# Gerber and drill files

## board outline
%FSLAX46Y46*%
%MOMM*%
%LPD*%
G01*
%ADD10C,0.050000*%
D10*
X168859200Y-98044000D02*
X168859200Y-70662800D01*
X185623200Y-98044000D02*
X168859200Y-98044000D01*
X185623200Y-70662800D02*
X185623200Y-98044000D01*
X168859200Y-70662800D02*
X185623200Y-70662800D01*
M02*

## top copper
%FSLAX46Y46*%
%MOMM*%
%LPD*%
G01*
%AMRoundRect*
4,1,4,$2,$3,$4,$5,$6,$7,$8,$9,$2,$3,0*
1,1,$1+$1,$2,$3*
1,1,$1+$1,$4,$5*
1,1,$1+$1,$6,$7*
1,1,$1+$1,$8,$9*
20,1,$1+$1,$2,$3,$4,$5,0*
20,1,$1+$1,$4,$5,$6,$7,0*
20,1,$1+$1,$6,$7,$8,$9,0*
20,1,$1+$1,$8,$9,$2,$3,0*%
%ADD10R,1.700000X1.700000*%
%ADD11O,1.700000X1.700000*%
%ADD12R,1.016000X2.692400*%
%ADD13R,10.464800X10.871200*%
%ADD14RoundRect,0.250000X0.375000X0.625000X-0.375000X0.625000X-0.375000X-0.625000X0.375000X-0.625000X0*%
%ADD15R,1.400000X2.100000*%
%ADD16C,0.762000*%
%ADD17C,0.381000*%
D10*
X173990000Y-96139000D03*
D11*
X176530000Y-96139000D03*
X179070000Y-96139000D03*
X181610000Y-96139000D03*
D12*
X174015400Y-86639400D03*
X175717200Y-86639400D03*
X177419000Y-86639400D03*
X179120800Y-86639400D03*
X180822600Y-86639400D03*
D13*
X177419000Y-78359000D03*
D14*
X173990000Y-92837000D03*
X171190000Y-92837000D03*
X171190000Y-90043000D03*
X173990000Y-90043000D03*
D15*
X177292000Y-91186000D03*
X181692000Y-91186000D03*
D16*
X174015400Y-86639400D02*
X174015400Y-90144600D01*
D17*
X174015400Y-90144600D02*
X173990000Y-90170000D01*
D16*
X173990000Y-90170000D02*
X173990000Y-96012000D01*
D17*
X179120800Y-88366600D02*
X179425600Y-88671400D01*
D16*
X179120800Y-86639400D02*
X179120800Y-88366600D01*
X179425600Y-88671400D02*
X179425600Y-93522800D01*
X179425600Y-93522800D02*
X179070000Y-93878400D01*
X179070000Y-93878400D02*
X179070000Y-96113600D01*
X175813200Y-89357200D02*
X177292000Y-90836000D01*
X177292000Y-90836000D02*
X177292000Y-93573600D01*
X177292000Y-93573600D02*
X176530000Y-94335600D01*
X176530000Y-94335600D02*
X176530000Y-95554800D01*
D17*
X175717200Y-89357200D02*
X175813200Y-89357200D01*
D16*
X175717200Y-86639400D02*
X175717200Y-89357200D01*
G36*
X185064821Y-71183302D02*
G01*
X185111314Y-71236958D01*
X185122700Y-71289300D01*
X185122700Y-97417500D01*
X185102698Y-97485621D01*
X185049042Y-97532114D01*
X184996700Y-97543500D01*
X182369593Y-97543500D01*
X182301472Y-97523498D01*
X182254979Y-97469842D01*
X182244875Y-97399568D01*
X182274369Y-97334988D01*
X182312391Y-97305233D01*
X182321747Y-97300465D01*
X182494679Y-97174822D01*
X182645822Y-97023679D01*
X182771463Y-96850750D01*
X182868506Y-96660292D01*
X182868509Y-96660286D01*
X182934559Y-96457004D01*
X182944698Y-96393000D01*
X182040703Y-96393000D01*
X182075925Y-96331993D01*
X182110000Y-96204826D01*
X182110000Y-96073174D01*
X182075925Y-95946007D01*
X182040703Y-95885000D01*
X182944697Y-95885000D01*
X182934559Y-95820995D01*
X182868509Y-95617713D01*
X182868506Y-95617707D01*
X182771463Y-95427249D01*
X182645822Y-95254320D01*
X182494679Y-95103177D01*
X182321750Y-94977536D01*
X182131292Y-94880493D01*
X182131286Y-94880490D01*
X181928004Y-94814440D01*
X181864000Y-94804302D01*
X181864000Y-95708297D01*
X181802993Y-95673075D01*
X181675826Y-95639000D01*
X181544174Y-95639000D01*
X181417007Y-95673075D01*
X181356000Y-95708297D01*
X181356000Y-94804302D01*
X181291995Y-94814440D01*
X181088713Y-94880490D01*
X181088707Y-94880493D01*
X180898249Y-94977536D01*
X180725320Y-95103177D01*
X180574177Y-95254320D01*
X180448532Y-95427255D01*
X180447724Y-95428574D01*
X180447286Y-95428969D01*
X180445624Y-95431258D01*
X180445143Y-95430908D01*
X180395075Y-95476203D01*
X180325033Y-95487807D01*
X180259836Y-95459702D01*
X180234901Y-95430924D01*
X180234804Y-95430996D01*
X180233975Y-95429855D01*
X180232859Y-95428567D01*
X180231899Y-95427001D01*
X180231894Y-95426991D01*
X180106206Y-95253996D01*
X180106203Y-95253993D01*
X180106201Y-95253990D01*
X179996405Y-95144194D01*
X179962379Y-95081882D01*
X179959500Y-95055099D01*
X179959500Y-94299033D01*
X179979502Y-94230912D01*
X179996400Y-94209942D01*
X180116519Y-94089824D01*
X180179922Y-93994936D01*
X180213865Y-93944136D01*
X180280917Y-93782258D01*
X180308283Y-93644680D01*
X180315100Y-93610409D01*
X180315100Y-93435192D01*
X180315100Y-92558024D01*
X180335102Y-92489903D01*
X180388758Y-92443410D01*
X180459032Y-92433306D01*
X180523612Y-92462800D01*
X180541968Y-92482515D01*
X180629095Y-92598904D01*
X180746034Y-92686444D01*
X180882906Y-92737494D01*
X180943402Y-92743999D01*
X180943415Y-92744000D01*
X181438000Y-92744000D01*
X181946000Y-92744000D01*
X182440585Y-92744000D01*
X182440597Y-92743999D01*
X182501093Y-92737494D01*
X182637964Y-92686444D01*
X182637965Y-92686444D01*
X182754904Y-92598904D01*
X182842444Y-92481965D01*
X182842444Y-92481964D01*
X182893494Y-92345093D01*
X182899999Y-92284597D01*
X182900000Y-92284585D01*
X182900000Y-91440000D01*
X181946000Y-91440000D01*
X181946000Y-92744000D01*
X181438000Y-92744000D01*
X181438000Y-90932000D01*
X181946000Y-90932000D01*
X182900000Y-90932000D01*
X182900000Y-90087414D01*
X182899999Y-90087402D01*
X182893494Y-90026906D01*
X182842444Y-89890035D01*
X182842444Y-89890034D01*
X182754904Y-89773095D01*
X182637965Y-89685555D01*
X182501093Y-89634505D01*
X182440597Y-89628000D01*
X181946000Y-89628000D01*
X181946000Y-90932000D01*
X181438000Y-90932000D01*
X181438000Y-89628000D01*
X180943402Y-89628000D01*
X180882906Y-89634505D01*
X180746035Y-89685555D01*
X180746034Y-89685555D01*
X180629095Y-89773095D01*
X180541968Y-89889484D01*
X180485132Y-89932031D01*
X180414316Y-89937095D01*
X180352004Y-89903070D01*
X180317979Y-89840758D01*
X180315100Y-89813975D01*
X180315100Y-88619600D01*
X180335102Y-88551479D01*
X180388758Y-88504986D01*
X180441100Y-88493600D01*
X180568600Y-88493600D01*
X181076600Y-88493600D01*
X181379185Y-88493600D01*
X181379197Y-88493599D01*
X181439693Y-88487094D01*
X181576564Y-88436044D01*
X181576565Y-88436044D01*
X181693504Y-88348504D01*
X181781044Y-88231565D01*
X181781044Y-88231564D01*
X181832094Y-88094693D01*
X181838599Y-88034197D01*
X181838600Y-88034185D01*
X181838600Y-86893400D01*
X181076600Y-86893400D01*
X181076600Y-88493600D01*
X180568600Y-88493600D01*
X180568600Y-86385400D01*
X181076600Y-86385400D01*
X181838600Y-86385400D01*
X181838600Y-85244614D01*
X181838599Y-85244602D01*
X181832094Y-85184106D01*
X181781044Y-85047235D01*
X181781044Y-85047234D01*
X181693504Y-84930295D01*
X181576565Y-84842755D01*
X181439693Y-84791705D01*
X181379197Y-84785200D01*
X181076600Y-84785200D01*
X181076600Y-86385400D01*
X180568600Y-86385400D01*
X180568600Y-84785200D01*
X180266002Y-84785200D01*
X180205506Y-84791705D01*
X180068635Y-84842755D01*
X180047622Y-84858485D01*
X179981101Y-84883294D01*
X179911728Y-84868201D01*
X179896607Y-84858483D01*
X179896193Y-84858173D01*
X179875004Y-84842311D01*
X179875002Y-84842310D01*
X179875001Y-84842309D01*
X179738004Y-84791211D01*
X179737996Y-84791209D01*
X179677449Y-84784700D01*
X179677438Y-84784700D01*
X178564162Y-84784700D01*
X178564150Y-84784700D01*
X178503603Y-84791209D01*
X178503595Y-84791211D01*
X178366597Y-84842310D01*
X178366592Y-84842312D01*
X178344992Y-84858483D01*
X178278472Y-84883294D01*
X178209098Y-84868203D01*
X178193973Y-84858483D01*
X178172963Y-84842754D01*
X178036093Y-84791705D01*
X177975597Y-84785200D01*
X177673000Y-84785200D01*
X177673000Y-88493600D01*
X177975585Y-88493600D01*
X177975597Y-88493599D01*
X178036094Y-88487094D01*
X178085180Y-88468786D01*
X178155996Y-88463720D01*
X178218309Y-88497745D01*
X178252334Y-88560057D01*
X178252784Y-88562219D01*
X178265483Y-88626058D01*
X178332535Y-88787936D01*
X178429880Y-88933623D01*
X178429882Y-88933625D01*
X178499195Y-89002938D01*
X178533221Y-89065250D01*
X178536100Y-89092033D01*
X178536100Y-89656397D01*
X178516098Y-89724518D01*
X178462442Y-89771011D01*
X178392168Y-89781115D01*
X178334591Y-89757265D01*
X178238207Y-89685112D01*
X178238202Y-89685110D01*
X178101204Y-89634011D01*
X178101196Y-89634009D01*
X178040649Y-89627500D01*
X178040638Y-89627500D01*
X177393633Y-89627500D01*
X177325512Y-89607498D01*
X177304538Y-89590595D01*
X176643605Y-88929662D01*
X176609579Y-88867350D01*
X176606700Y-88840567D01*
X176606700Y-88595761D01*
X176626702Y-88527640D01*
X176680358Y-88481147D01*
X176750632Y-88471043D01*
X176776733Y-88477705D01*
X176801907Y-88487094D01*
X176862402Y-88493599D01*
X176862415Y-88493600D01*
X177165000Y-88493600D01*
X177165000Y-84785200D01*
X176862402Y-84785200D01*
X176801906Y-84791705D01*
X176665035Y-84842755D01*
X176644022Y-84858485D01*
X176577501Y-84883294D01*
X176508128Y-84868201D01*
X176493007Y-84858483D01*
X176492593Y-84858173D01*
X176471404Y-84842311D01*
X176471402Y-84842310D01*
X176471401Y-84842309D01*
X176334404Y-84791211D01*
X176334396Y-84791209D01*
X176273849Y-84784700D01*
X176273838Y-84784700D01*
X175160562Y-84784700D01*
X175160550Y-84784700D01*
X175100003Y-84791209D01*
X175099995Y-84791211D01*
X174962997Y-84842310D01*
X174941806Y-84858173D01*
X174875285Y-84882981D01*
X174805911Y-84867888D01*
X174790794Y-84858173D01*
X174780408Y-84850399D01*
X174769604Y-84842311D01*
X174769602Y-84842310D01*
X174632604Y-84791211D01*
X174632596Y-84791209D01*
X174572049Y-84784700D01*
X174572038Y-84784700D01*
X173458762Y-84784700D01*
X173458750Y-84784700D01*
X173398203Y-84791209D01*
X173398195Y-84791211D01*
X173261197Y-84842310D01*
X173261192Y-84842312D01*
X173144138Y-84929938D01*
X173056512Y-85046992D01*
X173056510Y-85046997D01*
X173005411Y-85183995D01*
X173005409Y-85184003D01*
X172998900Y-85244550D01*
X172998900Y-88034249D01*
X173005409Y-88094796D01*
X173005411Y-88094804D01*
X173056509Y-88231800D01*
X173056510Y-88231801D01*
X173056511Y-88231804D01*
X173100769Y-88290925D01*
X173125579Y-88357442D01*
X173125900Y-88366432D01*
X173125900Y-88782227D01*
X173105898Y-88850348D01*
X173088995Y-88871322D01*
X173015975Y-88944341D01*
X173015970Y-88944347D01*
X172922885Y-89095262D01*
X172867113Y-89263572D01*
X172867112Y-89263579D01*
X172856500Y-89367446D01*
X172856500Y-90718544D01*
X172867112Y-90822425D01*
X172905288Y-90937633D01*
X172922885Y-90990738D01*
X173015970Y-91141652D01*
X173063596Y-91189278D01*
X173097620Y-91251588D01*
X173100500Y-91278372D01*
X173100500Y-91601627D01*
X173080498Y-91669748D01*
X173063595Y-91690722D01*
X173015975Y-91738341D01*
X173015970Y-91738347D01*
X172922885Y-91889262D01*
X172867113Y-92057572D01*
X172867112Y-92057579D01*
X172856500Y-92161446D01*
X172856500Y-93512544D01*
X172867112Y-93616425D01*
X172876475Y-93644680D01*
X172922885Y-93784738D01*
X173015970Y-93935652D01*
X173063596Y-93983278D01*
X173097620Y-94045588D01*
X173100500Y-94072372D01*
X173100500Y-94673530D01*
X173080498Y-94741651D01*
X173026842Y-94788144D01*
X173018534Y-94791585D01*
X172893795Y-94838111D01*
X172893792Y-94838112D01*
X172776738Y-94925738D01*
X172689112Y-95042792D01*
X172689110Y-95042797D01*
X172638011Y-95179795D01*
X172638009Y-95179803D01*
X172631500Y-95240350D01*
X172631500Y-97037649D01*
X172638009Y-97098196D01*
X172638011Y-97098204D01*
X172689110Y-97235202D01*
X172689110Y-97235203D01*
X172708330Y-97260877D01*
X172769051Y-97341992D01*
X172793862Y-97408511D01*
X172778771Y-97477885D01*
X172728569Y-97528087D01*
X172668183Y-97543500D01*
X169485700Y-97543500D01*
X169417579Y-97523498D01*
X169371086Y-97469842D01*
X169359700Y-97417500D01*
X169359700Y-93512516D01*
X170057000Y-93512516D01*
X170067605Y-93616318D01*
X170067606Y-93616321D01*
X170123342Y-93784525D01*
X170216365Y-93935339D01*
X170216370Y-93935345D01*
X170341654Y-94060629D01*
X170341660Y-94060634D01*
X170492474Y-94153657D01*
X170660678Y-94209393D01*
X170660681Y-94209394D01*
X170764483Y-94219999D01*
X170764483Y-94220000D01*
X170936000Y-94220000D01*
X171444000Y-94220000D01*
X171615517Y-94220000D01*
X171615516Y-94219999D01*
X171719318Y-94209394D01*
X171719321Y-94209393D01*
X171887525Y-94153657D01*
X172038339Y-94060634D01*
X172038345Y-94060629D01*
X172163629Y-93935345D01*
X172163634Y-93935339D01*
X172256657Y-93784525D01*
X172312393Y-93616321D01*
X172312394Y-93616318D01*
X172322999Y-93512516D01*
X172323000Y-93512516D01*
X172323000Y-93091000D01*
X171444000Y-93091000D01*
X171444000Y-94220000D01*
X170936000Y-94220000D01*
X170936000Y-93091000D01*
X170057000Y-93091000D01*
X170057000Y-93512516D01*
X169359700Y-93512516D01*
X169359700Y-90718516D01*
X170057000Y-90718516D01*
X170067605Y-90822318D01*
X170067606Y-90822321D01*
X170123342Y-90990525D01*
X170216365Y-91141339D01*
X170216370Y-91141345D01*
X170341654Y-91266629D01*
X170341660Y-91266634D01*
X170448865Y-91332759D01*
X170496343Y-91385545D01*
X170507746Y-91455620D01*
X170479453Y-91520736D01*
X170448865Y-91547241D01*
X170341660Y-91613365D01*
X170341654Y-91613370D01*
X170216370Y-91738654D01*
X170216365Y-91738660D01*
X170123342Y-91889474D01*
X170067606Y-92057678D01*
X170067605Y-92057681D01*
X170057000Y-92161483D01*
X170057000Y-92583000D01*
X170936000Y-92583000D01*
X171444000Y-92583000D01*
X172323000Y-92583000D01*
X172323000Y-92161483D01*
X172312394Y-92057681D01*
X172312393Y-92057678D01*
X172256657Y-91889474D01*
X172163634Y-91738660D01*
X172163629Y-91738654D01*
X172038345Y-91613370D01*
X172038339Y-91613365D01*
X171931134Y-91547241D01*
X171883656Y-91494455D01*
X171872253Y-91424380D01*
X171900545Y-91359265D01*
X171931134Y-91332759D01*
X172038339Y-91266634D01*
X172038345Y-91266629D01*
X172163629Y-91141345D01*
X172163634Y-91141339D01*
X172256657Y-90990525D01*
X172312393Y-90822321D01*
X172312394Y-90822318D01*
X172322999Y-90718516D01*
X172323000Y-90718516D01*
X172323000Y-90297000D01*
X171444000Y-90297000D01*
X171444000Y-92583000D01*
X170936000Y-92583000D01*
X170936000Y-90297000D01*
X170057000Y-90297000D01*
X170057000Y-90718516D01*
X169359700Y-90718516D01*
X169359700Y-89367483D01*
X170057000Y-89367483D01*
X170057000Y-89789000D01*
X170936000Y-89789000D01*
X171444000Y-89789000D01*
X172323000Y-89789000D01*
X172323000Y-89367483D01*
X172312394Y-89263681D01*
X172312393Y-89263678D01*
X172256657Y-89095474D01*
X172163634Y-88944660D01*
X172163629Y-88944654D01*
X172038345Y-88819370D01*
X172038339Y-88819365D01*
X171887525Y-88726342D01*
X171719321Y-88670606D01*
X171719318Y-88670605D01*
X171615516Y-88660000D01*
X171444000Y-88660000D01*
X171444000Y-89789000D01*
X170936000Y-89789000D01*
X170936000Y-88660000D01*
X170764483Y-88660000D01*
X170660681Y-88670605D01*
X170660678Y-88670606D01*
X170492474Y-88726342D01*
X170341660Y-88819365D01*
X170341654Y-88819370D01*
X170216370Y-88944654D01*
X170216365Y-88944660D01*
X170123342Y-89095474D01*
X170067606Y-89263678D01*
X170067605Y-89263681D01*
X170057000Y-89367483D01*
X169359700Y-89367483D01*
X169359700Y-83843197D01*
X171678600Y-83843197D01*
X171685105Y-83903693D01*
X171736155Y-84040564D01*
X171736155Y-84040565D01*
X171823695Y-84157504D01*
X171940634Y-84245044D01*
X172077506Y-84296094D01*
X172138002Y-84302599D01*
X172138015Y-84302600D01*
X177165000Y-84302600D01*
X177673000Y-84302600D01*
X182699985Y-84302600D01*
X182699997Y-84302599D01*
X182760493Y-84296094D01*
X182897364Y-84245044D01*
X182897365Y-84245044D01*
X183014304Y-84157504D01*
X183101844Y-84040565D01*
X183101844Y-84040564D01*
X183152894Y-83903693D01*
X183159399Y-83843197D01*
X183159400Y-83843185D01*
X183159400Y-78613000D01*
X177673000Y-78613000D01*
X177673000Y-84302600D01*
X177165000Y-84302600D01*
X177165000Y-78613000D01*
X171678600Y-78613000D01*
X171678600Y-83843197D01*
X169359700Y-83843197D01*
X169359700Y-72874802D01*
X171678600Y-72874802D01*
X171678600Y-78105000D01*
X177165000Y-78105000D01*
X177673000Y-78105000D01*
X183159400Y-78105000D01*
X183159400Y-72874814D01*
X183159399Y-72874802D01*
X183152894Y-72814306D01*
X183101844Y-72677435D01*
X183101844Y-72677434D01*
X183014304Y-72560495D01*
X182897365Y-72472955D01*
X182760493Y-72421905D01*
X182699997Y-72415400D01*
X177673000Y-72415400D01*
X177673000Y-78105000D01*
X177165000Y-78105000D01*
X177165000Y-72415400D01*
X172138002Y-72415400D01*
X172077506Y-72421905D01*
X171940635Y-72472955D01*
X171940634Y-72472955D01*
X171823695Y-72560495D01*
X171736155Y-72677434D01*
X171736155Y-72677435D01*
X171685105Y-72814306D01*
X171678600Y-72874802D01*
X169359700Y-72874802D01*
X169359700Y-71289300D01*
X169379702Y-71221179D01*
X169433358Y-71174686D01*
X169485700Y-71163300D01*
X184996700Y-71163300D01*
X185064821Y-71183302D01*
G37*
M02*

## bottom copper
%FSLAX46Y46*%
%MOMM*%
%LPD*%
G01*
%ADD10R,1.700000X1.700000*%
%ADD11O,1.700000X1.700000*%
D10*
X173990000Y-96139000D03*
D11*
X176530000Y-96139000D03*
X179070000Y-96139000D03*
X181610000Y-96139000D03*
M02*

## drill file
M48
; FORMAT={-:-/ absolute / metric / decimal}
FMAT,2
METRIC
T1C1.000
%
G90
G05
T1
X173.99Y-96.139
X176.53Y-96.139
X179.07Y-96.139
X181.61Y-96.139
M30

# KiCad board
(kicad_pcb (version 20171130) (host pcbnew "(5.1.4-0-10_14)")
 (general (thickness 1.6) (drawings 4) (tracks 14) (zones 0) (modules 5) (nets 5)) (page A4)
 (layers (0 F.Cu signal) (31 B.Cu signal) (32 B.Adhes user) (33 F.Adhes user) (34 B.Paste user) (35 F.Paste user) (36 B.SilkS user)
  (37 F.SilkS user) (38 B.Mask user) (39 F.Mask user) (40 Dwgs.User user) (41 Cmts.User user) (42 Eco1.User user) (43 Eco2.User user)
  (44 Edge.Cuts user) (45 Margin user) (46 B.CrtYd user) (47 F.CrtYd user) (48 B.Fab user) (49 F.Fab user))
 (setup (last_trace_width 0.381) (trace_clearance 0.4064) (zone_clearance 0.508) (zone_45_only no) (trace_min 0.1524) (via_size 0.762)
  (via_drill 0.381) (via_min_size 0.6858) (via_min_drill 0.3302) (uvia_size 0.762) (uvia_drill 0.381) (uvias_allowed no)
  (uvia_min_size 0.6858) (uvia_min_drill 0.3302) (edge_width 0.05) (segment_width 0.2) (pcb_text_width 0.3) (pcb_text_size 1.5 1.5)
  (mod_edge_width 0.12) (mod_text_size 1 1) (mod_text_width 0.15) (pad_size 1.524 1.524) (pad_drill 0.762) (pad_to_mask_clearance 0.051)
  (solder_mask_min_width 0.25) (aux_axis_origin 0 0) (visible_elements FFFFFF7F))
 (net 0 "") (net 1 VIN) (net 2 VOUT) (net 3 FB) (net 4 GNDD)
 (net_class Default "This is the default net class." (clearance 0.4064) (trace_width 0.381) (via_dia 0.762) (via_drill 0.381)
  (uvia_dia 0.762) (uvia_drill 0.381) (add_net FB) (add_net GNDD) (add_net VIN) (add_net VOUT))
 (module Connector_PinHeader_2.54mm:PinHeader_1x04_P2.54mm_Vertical (layer F.Cu) (at 173.99 96.139 90)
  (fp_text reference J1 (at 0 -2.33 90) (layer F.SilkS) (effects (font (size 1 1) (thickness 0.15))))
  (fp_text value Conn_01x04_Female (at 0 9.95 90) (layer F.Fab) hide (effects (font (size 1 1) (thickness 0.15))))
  (pad 1 thru_hole rect (at 0 0 90) (size 1.7 1.7) (drill 1) (layers *.Cu *.Mask) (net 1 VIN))
  (pad 2 thru_hole oval (at 0 2.54 90) (size 1.7 1.7) (drill 1) (layers *.Cu *.Mask) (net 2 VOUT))
  (pad 3 thru_hole oval (at 0 5.08 90) (size 1.7 1.7) (drill 1) (layers *.Cu *.Mask) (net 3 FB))
  (pad 4 thru_hole oval (at 0 7.62 90) (size 1.7 1.7) (drill 1) (layers *.Cu *.Mask) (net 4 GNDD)))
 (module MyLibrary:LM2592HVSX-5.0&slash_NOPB (layer F.Cu) (at 177.419 78.359)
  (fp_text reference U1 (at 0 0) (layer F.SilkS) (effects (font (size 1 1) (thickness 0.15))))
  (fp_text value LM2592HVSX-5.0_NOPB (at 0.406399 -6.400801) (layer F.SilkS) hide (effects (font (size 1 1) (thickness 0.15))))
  (pad 1 smd rect (at -3.4036 8.2804) (size 1.016 2.6924) (layers F.Cu F.Paste F.Mask) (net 1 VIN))
  (pad 2 smd rect (at -1.7018 8.2804) (size 1.016 2.6924) (layers F.Cu F.Paste F.Mask) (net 2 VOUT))
  (pad 3 smd rect (at 0 8.2804) (size 1.016 2.6924) (layers F.Cu F.Paste F.Mask) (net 4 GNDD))
  (pad 4 smd rect (at 1.7018 8.2804) (size 1.016 2.6924) (layers F.Cu F.Paste F.Mask) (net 3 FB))
  (pad 5 smd rect (at 3.4036 8.2804) (size 1.016 2.6924) (layers F.Cu F.Paste F.Mask) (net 4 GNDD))
  (pad 6 smd rect (at 0 0) (size 10.4648 10.8712) (layers F.Cu F.Paste F.Mask) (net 4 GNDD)))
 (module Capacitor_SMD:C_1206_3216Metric (layer F.Cu) (at 172.59 92.837 180)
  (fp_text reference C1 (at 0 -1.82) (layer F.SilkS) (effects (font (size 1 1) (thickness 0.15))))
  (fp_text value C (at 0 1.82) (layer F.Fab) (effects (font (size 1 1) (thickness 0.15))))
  (pad 1 smd roundrect (at -1.4 0 180) (size 1.25 1.75) (layers F.Cu F.Paste F.Mask) (roundrect_rratio 0.2) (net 1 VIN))
  (pad 2 smd roundrect (at 1.4 0 180) (size 1.25 1.75) (layers F.Cu F.Paste F.Mask) (roundrect_rratio 0.2) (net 4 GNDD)))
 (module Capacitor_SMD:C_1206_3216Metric (layer F.Cu) (at 172.59 90.043 180)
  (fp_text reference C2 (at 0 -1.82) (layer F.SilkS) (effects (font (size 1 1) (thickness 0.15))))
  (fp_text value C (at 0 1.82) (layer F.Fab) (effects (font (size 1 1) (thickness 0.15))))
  (pad 2 smd roundrect (at 1.4 0 180) (size 1.25 1.75) (layers F.Cu F.Paste F.Mask) (roundrect_rratio 0.2) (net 4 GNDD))
  (pad 1 smd roundrect (at -1.4 0 180) (size 1.25 1.75) (layers F.Cu F.Paste F.Mask) (roundrect_rratio 0.2) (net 1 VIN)))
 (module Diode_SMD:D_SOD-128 (layer F.Cu) (at 179.492 91.186)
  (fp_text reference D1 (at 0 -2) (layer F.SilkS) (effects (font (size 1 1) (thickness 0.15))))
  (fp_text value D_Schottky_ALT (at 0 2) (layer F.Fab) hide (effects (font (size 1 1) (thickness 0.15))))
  (pad 1 smd rect (at -2.2 0) (size 1.4 2.1) (layers F.Cu F.Paste F.Mask) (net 2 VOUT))
  (pad 2 smd rect (at 2.2 0) (size 1.4 2.1) (layers F.Cu F.Paste F.Mask) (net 4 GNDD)))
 (gr_line (start 168.8592 98.044) (end 168.8592 70.6628) (layer Edge.Cuts) (width 0.05))
 (gr_line (start 185.6232 98.044) (end 168.8592 98.044) (layer Edge.Cuts) (width 0.05))
 (gr_line (start 185.6232 70.6628) (end 185.6232 98.044) (layer Edge.Cuts) (width 0.05))
 (gr_line (start 168.8592 70.6628) (end 185.6232 70.6628) (layer Edge.Cuts) (width 0.05))
 (segment (start 174.0154 86.6394) (end 174.0154 90.1446) (width 0.762) (layer F.Cu) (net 1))
 (segment (start 174.0154 90.1446) (end 173.99 90.17) (width 0.381) (layer F.Cu) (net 1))
 (segment (start 173.99 90.17) (end 173.99 96.012) (width 0.762) (layer F.Cu) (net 1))
 (segment (start 179.1208 88.3666) (end 179.4256 88.6714) (width 0.381) (layer F.Cu) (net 3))
 (segment (start 179.1208 86.6394) (end 179.1208 88.3666) (width 0.762) (layer F.Cu) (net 3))
 (segment (start 179.4256 88.6714) (end 179.4256 93.5228) (width 0.762) (layer F.Cu) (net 3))
 (segment (start 179.4256 93.5228) (end 179.07 93.8784) (width 0.762) (layer F.Cu) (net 3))
 (segment (start 179.07 93.8784) (end 179.07 96.1136) (width 0.762) (layer F.Cu) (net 3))
 (segment (start 175.8132 89.3572) (end 177.292 90.836) (width 0.762) (layer F.Cu) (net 2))
 (segment (start 177.292 90.836) (end 177.292 93.5736) (width 0.762) (layer F.Cu) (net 2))
 (segment (start 177.292 93.5736) (end 176.53 94.3356) (width 0.762) (layer F.Cu) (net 2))
 (segment (start 176.53 94.3356) (end 176.53 95.5548) (width 0.762) (layer F.Cu) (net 2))
 (segment (start 175.7172 89.3572) (end 175.8132 89.3572) (width 0.381) (layer F.Cu) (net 2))
 (segment (start 175.7172 86.6394) (end 175.7172 89.3572) (width 0.762) (layer F.Cu) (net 2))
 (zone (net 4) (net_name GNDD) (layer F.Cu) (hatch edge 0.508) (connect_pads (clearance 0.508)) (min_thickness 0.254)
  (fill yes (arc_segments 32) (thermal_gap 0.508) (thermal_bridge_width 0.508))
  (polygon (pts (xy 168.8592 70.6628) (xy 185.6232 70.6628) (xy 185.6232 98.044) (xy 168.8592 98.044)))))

